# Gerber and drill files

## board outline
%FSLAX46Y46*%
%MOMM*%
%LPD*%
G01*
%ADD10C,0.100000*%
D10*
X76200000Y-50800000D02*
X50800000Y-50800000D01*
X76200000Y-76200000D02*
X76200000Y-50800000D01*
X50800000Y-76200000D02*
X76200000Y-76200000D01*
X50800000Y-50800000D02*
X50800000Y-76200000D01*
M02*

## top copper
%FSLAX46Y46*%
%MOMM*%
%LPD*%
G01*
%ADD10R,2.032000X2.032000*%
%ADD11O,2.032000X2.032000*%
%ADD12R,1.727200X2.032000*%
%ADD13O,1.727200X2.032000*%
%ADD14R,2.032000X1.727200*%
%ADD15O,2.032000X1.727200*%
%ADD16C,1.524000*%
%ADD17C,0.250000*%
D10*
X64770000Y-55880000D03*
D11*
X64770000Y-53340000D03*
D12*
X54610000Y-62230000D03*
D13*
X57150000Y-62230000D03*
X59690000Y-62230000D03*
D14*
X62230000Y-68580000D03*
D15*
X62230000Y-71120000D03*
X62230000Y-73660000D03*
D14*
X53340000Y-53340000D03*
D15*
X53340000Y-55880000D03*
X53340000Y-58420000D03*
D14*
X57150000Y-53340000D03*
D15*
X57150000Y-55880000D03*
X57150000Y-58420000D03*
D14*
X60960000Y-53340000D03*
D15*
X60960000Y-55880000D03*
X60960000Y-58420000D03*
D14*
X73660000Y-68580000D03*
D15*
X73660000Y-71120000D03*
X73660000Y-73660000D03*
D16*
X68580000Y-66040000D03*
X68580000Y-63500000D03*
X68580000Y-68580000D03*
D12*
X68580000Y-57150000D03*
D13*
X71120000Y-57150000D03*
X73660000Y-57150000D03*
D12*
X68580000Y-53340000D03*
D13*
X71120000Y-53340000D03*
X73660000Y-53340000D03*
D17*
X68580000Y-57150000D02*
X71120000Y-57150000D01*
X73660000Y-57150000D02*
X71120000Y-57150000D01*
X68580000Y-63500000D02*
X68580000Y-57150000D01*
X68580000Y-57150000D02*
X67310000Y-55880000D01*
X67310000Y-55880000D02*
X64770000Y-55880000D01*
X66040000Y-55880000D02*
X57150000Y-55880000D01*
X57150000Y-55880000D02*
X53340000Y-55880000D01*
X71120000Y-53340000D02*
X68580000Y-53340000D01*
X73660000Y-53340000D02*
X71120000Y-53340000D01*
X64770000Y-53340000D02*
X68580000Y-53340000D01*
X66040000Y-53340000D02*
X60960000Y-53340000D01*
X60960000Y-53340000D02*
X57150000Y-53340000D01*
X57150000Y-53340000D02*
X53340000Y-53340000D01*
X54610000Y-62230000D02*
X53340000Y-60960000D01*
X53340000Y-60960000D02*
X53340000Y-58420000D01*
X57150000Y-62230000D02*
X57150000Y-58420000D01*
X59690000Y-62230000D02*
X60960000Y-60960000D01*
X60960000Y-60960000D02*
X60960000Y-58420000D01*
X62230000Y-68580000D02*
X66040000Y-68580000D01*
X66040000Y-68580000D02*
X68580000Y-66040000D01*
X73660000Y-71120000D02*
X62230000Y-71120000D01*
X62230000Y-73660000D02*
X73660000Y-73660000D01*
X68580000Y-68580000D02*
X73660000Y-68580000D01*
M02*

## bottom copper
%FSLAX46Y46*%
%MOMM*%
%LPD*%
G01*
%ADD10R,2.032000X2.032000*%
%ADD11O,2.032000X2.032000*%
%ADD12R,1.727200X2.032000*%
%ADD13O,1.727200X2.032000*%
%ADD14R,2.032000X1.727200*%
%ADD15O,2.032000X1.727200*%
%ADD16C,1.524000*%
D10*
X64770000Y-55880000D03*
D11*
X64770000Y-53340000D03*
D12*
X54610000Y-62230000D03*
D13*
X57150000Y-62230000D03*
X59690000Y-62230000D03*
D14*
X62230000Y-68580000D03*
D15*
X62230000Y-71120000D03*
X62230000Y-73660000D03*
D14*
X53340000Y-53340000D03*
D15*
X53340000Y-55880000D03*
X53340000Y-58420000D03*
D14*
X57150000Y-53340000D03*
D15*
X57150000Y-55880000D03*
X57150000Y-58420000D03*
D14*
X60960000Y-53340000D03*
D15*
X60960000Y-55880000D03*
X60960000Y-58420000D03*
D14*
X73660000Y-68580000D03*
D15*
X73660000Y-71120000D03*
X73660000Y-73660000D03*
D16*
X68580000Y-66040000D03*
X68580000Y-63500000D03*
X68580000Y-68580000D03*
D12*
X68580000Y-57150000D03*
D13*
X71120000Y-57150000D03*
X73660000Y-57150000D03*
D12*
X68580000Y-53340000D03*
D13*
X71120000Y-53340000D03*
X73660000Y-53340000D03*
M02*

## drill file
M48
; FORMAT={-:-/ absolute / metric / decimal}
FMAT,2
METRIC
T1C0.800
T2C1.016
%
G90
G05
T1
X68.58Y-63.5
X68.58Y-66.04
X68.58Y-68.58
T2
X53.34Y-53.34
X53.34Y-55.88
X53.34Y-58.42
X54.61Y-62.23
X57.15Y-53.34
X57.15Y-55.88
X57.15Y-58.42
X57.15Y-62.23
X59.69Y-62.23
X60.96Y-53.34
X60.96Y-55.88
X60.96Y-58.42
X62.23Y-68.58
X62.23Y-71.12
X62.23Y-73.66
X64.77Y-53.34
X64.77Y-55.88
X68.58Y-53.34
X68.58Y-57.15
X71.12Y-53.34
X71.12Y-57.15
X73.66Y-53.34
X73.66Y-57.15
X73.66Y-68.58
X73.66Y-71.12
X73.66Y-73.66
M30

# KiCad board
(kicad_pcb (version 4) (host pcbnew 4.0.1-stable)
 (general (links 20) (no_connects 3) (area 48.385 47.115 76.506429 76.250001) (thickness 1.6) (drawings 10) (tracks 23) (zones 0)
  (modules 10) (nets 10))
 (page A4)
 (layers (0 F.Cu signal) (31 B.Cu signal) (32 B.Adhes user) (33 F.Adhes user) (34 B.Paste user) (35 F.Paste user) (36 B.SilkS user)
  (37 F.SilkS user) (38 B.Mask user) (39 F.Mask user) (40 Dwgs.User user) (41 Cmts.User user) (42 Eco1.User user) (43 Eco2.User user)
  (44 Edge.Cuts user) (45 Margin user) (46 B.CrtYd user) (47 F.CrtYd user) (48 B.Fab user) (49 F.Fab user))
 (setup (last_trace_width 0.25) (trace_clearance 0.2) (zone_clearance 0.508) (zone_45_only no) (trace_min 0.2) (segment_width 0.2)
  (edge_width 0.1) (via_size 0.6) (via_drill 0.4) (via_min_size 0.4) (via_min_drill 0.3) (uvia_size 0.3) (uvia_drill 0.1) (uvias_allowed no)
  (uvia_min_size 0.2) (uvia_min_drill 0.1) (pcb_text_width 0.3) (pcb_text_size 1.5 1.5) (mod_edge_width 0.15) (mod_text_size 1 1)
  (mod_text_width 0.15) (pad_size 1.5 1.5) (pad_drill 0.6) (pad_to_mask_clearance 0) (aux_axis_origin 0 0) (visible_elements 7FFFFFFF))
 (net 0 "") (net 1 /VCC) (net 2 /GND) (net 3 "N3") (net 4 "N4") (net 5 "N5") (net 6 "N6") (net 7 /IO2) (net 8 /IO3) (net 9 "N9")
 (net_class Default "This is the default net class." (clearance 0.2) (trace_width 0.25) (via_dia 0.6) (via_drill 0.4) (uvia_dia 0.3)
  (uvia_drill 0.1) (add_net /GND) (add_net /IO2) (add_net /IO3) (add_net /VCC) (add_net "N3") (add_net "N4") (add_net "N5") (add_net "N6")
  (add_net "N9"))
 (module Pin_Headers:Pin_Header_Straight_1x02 (layer F.Cu) (at 64.77 55.88 180)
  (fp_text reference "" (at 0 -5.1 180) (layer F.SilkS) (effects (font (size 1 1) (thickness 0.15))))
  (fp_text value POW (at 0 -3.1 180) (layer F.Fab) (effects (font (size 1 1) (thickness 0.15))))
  (pad 1 thru_hole rect (at 0 0 180) (size 2.032 2.032) (drill 1.016) (layers *.Cu *.Mask F.SilkS) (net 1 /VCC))
  (pad 2 thru_hole oval (at 0 2.54 180) (size 2.032 2.032) (drill 1.016) (layers *.Cu *.Mask F.SilkS) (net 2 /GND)))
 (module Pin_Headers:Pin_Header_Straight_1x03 (layer F.Cu) (at 54.61 62.23 90)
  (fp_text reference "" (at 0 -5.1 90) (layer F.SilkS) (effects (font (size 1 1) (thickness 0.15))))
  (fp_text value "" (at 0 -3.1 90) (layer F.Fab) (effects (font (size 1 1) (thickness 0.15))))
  (pad 1 thru_hole rect (at 0 0 90) (size 2.032 1.7272) (drill 1.016) (layers *.Cu *.Mask F.SilkS) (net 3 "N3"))
  (pad 2 thru_hole oval (at 0 2.54 90) (size 2.032 1.7272) (drill 1.016) (layers *.Cu *.Mask F.SilkS) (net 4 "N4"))
  (pad 3 thru_hole oval (at 0 5.08 90) (size 2.032 1.7272) (drill 1.016) (layers *.Cu *.Mask F.SilkS) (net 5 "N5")))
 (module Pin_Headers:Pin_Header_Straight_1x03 (layer F.Cu) (at 62.23 68.58)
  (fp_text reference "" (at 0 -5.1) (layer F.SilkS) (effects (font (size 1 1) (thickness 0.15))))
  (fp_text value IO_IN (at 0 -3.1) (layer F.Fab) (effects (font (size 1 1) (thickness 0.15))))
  (pad 1 thru_hole rect (at 0 0) (size 2.032 1.7272) (drill 1.016) (layers *.Cu *.Mask F.SilkS) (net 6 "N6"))
  (pad 2 thru_hole oval (at 0 2.54) (size 2.032 1.7272) (drill 1.016) (layers *.Cu *.Mask F.SilkS) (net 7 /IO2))
  (pad 3 thru_hole oval (at 0 5.08) (size 2.032 1.7272) (drill 1.016) (layers *.Cu *.Mask F.SilkS) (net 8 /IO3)))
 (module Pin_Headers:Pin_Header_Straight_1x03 (layer F.Cu) (at 53.34 53.34)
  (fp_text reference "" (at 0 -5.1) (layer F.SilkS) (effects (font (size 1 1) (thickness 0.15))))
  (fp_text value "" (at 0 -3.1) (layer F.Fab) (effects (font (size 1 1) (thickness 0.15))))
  (pad 1 thru_hole rect (at 0 0) (size 2.032 1.7272) (drill 1.016) (layers *.Cu *.Mask F.SilkS) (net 2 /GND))
  (pad 2 thru_hole oval (at 0 2.54) (size 2.032 1.7272) (drill 1.016) (layers *.Cu *.Mask F.SilkS) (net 1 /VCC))
  (pad 3 thru_hole oval (at 0 5.08) (size 2.032 1.7272) (drill 1.016) (layers *.Cu *.Mask F.SilkS) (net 3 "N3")))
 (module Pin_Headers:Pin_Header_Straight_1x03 (layer F.Cu) (at 57.15 53.34)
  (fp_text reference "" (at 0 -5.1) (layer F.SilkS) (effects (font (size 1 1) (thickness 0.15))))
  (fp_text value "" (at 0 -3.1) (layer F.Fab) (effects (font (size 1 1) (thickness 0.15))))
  (pad 1 thru_hole rect (at 0 0) (size 2.032 1.7272) (drill 1.016) (layers *.Cu *.Mask F.SilkS) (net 2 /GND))
  (pad 2 thru_hole oval (at 0 2.54) (size 2.032 1.7272) (drill 1.016) (layers *.Cu *.Mask F.SilkS) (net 1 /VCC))
  (pad 3 thru_hole oval (at 0 5.08) (size 2.032 1.7272) (drill 1.016) (layers *.Cu *.Mask F.SilkS) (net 4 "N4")))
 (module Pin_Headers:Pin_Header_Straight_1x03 (layer F.Cu) (at 60.96 53.34)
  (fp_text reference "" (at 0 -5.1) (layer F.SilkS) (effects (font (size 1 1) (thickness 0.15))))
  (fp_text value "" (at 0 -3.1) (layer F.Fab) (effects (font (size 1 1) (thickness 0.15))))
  (pad 1 thru_hole rect (at 0 0) (size 2.032 1.7272) (drill 1.016) (layers *.Cu *.Mask F.SilkS) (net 2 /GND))
  (pad 2 thru_hole oval (at 0 2.54) (size 2.032 1.7272) (drill 1.016) (layers *.Cu *.Mask F.SilkS) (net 1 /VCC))
  (pad 3 thru_hole oval (at 0 5.08) (size 2.032 1.7272) (drill 1.016) (layers *.Cu *.Mask F.SilkS) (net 5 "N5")))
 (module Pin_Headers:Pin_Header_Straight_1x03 (layer F.Cu) (at 73.66 68.58)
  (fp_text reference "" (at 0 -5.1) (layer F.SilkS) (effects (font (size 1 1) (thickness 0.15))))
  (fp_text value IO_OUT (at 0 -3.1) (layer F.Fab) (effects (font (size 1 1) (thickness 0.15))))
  (pad 1 thru_hole rect (at 0 0) (size 2.032 1.7272) (drill 1.016) (layers *.Cu *.Mask F.SilkS) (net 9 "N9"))
  (pad 2 thru_hole oval (at 0 2.54) (size 2.032 1.7272) (drill 1.016) (layers *.Cu *.Mask F.SilkS) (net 7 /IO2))
  (pad 3 thru_hole oval (at 0 5.08) (size 2.032 1.7272) (drill 1.016) (layers *.Cu *.Mask F.SilkS) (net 8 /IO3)))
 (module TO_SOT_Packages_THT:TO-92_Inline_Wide (layer F.Cu) (at 68.58 68.58 90)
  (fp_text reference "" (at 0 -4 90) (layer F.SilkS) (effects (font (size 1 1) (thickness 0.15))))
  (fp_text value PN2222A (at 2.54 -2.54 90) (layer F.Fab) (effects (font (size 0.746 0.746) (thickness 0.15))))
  (pad 2 thru_hole circle (at 2.54 0 180) (size 1.524 1.524) (drill 0.8) (layers *.Cu *.Mask F.SilkS) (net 6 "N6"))
  (pad 3 thru_hole circle (at 5.08 0 180) (size 1.524 1.524) (drill 0.8) (layers *.Cu *.Mask F.SilkS) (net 1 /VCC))
  (pad 1 thru_hole circle (at 0 0 180) (size 1.524 1.524) (drill 0.8) (layers *.Cu *.Mask F.SilkS) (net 9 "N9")))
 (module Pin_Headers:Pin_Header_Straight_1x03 (layer F.Cu) (at 68.58 57.15 90)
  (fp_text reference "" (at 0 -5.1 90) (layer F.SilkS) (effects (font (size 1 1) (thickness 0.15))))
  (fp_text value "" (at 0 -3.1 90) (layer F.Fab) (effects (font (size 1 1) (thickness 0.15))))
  (pad 1 thru_hole rect (at 0 0 90) (size 2.032 1.7272) (drill 1.016) (layers *.Cu *.Mask F.SilkS) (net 1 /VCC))
  (pad 2 thru_hole oval (at 0 2.54 90) (size 2.032 1.7272) (drill 1.016) (layers *.Cu *.Mask F.SilkS) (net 1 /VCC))
  (pad 3 thru_hole oval (at 0 5.08 90) (size 2.032 1.7272) (drill 1.016) (layers *.Cu *.Mask F.SilkS) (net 1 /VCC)))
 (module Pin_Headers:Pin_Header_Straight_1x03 (layer F.Cu) (at 68.58 53.34 90)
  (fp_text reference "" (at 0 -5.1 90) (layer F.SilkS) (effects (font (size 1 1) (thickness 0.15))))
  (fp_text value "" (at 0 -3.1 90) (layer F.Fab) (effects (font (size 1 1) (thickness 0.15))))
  (pad 1 thru_hole rect (at 0 0 90) (size 2.032 1.7272) (drill 1.016) (layers *.Cu *.Mask F.SilkS) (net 2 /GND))
  (pad 2 thru_hole oval (at 0 2.54 90) (size 2.032 1.7272) (drill 1.016) (layers *.Cu *.Mask F.SilkS) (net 2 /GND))
  (pad 3 thru_hole oval (at 0 5.08 90) (size 2.032 1.7272) (drill 1.016) (layers *.Cu *.Mask F.SilkS) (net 2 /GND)))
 (gr_line (start 76.2 50.8) (end 50.8 50.8) (angle 90) (layer Edge.Cuts) (width 0.1))
 (gr_line (start 76.2 76.2) (end 76.2 50.8) (angle 90) (layer Edge.Cuts) (width 0.1))
 (gr_line (start 50.8 76.2) (end 76.2 76.2) (angle 90) (layer Edge.Cuts) (width 0.1))
 (gr_line (start 50.8 50.8) (end 50.8 76.2) (angle 90) (layer Edge.Cuts) (width 0.1))
 (segment (start 68.58 57.15) (end 71.12 57.15) (width 0.25) (layer F.Cu) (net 1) (status 30))
 (segment (start 73.66 57.15) (end 71.12 57.15) (width 0.25) (layer F.Cu) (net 1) (status 30))
 (segment (start 68.58 63.5) (end 68.58 57.15) (width 0.25) (layer F.Cu) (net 1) (status 20))
 (segment (start 68.58 57.15) (end 67.31 55.88) (width 0.25) (layer F.Cu) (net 1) (status 10))
 (segment (start 67.31 55.88) (end 64.77 55.88) (width 0.25) (layer F.Cu) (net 1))
 (segment (start 66.04 55.88) (end 57.15 55.88) (width 0.25) (layer F.Cu) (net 1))
 (segment (start 57.15 55.88) (end 53.34 55.88) (width 0.25) (layer F.Cu) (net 1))
 (segment (start 71.12 53.34) (end 68.58 53.34) (width 0.25) (layer F.Cu) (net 2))
 (segment (start 73.66 53.34) (end 71.12 53.34) (width 0.25) (layer F.Cu) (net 2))
 (segment (start 64.77 53.34) (end 68.58 53.34) (width 0.25) (layer F.Cu) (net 2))
 (segment (start 66.04 53.34) (end 60.96 53.34) (width 0.25) (layer F.Cu) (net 2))
 (segment (start 60.96 53.34) (end 57.15 53.34) (width 0.25) (layer F.Cu) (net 2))
 (segment (start 57.15 53.34) (end 53.34 53.34) (width 0.25) (layer F.Cu) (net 2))
 (segment (start 54.61 62.23) (end 53.34 60.96) (width 0.25) (layer F.Cu) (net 3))
 (segment (start 53.34 60.96) (end 53.34 58.42) (width 0.25) (layer F.Cu) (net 3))
 (segment (start 57.15 62.23) (end 57.15 58.42) (width 0.25) (layer F.Cu) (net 4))
 (segment (start 59.69 62.23) (end 60.96 60.96) (width 0.25) (layer F.Cu) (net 5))
 (segment (start 60.96 60.96) (end 60.96 58.42) (width 0.25) (layer F.Cu) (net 5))
 (segment (start 62.23 68.58) (end 66.04 68.58) (width 0.25) (layer F.Cu) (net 6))
 (segment (start 66.04 68.58) (end 68.58 66.04) (width 0.25) (layer F.Cu) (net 6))
 (segment (start 73.66 71.12) (end 62.23 71.12) (width 0.25) (layer F.Cu) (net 7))
 (segment (start 62.23 73.66) (end 73.66 73.66) (width 0.25) (layer F.Cu) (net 8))
 (segment (start 68.58 68.58) (end 73.66 68.58) (width 0.25) (layer F.Cu) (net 9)))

